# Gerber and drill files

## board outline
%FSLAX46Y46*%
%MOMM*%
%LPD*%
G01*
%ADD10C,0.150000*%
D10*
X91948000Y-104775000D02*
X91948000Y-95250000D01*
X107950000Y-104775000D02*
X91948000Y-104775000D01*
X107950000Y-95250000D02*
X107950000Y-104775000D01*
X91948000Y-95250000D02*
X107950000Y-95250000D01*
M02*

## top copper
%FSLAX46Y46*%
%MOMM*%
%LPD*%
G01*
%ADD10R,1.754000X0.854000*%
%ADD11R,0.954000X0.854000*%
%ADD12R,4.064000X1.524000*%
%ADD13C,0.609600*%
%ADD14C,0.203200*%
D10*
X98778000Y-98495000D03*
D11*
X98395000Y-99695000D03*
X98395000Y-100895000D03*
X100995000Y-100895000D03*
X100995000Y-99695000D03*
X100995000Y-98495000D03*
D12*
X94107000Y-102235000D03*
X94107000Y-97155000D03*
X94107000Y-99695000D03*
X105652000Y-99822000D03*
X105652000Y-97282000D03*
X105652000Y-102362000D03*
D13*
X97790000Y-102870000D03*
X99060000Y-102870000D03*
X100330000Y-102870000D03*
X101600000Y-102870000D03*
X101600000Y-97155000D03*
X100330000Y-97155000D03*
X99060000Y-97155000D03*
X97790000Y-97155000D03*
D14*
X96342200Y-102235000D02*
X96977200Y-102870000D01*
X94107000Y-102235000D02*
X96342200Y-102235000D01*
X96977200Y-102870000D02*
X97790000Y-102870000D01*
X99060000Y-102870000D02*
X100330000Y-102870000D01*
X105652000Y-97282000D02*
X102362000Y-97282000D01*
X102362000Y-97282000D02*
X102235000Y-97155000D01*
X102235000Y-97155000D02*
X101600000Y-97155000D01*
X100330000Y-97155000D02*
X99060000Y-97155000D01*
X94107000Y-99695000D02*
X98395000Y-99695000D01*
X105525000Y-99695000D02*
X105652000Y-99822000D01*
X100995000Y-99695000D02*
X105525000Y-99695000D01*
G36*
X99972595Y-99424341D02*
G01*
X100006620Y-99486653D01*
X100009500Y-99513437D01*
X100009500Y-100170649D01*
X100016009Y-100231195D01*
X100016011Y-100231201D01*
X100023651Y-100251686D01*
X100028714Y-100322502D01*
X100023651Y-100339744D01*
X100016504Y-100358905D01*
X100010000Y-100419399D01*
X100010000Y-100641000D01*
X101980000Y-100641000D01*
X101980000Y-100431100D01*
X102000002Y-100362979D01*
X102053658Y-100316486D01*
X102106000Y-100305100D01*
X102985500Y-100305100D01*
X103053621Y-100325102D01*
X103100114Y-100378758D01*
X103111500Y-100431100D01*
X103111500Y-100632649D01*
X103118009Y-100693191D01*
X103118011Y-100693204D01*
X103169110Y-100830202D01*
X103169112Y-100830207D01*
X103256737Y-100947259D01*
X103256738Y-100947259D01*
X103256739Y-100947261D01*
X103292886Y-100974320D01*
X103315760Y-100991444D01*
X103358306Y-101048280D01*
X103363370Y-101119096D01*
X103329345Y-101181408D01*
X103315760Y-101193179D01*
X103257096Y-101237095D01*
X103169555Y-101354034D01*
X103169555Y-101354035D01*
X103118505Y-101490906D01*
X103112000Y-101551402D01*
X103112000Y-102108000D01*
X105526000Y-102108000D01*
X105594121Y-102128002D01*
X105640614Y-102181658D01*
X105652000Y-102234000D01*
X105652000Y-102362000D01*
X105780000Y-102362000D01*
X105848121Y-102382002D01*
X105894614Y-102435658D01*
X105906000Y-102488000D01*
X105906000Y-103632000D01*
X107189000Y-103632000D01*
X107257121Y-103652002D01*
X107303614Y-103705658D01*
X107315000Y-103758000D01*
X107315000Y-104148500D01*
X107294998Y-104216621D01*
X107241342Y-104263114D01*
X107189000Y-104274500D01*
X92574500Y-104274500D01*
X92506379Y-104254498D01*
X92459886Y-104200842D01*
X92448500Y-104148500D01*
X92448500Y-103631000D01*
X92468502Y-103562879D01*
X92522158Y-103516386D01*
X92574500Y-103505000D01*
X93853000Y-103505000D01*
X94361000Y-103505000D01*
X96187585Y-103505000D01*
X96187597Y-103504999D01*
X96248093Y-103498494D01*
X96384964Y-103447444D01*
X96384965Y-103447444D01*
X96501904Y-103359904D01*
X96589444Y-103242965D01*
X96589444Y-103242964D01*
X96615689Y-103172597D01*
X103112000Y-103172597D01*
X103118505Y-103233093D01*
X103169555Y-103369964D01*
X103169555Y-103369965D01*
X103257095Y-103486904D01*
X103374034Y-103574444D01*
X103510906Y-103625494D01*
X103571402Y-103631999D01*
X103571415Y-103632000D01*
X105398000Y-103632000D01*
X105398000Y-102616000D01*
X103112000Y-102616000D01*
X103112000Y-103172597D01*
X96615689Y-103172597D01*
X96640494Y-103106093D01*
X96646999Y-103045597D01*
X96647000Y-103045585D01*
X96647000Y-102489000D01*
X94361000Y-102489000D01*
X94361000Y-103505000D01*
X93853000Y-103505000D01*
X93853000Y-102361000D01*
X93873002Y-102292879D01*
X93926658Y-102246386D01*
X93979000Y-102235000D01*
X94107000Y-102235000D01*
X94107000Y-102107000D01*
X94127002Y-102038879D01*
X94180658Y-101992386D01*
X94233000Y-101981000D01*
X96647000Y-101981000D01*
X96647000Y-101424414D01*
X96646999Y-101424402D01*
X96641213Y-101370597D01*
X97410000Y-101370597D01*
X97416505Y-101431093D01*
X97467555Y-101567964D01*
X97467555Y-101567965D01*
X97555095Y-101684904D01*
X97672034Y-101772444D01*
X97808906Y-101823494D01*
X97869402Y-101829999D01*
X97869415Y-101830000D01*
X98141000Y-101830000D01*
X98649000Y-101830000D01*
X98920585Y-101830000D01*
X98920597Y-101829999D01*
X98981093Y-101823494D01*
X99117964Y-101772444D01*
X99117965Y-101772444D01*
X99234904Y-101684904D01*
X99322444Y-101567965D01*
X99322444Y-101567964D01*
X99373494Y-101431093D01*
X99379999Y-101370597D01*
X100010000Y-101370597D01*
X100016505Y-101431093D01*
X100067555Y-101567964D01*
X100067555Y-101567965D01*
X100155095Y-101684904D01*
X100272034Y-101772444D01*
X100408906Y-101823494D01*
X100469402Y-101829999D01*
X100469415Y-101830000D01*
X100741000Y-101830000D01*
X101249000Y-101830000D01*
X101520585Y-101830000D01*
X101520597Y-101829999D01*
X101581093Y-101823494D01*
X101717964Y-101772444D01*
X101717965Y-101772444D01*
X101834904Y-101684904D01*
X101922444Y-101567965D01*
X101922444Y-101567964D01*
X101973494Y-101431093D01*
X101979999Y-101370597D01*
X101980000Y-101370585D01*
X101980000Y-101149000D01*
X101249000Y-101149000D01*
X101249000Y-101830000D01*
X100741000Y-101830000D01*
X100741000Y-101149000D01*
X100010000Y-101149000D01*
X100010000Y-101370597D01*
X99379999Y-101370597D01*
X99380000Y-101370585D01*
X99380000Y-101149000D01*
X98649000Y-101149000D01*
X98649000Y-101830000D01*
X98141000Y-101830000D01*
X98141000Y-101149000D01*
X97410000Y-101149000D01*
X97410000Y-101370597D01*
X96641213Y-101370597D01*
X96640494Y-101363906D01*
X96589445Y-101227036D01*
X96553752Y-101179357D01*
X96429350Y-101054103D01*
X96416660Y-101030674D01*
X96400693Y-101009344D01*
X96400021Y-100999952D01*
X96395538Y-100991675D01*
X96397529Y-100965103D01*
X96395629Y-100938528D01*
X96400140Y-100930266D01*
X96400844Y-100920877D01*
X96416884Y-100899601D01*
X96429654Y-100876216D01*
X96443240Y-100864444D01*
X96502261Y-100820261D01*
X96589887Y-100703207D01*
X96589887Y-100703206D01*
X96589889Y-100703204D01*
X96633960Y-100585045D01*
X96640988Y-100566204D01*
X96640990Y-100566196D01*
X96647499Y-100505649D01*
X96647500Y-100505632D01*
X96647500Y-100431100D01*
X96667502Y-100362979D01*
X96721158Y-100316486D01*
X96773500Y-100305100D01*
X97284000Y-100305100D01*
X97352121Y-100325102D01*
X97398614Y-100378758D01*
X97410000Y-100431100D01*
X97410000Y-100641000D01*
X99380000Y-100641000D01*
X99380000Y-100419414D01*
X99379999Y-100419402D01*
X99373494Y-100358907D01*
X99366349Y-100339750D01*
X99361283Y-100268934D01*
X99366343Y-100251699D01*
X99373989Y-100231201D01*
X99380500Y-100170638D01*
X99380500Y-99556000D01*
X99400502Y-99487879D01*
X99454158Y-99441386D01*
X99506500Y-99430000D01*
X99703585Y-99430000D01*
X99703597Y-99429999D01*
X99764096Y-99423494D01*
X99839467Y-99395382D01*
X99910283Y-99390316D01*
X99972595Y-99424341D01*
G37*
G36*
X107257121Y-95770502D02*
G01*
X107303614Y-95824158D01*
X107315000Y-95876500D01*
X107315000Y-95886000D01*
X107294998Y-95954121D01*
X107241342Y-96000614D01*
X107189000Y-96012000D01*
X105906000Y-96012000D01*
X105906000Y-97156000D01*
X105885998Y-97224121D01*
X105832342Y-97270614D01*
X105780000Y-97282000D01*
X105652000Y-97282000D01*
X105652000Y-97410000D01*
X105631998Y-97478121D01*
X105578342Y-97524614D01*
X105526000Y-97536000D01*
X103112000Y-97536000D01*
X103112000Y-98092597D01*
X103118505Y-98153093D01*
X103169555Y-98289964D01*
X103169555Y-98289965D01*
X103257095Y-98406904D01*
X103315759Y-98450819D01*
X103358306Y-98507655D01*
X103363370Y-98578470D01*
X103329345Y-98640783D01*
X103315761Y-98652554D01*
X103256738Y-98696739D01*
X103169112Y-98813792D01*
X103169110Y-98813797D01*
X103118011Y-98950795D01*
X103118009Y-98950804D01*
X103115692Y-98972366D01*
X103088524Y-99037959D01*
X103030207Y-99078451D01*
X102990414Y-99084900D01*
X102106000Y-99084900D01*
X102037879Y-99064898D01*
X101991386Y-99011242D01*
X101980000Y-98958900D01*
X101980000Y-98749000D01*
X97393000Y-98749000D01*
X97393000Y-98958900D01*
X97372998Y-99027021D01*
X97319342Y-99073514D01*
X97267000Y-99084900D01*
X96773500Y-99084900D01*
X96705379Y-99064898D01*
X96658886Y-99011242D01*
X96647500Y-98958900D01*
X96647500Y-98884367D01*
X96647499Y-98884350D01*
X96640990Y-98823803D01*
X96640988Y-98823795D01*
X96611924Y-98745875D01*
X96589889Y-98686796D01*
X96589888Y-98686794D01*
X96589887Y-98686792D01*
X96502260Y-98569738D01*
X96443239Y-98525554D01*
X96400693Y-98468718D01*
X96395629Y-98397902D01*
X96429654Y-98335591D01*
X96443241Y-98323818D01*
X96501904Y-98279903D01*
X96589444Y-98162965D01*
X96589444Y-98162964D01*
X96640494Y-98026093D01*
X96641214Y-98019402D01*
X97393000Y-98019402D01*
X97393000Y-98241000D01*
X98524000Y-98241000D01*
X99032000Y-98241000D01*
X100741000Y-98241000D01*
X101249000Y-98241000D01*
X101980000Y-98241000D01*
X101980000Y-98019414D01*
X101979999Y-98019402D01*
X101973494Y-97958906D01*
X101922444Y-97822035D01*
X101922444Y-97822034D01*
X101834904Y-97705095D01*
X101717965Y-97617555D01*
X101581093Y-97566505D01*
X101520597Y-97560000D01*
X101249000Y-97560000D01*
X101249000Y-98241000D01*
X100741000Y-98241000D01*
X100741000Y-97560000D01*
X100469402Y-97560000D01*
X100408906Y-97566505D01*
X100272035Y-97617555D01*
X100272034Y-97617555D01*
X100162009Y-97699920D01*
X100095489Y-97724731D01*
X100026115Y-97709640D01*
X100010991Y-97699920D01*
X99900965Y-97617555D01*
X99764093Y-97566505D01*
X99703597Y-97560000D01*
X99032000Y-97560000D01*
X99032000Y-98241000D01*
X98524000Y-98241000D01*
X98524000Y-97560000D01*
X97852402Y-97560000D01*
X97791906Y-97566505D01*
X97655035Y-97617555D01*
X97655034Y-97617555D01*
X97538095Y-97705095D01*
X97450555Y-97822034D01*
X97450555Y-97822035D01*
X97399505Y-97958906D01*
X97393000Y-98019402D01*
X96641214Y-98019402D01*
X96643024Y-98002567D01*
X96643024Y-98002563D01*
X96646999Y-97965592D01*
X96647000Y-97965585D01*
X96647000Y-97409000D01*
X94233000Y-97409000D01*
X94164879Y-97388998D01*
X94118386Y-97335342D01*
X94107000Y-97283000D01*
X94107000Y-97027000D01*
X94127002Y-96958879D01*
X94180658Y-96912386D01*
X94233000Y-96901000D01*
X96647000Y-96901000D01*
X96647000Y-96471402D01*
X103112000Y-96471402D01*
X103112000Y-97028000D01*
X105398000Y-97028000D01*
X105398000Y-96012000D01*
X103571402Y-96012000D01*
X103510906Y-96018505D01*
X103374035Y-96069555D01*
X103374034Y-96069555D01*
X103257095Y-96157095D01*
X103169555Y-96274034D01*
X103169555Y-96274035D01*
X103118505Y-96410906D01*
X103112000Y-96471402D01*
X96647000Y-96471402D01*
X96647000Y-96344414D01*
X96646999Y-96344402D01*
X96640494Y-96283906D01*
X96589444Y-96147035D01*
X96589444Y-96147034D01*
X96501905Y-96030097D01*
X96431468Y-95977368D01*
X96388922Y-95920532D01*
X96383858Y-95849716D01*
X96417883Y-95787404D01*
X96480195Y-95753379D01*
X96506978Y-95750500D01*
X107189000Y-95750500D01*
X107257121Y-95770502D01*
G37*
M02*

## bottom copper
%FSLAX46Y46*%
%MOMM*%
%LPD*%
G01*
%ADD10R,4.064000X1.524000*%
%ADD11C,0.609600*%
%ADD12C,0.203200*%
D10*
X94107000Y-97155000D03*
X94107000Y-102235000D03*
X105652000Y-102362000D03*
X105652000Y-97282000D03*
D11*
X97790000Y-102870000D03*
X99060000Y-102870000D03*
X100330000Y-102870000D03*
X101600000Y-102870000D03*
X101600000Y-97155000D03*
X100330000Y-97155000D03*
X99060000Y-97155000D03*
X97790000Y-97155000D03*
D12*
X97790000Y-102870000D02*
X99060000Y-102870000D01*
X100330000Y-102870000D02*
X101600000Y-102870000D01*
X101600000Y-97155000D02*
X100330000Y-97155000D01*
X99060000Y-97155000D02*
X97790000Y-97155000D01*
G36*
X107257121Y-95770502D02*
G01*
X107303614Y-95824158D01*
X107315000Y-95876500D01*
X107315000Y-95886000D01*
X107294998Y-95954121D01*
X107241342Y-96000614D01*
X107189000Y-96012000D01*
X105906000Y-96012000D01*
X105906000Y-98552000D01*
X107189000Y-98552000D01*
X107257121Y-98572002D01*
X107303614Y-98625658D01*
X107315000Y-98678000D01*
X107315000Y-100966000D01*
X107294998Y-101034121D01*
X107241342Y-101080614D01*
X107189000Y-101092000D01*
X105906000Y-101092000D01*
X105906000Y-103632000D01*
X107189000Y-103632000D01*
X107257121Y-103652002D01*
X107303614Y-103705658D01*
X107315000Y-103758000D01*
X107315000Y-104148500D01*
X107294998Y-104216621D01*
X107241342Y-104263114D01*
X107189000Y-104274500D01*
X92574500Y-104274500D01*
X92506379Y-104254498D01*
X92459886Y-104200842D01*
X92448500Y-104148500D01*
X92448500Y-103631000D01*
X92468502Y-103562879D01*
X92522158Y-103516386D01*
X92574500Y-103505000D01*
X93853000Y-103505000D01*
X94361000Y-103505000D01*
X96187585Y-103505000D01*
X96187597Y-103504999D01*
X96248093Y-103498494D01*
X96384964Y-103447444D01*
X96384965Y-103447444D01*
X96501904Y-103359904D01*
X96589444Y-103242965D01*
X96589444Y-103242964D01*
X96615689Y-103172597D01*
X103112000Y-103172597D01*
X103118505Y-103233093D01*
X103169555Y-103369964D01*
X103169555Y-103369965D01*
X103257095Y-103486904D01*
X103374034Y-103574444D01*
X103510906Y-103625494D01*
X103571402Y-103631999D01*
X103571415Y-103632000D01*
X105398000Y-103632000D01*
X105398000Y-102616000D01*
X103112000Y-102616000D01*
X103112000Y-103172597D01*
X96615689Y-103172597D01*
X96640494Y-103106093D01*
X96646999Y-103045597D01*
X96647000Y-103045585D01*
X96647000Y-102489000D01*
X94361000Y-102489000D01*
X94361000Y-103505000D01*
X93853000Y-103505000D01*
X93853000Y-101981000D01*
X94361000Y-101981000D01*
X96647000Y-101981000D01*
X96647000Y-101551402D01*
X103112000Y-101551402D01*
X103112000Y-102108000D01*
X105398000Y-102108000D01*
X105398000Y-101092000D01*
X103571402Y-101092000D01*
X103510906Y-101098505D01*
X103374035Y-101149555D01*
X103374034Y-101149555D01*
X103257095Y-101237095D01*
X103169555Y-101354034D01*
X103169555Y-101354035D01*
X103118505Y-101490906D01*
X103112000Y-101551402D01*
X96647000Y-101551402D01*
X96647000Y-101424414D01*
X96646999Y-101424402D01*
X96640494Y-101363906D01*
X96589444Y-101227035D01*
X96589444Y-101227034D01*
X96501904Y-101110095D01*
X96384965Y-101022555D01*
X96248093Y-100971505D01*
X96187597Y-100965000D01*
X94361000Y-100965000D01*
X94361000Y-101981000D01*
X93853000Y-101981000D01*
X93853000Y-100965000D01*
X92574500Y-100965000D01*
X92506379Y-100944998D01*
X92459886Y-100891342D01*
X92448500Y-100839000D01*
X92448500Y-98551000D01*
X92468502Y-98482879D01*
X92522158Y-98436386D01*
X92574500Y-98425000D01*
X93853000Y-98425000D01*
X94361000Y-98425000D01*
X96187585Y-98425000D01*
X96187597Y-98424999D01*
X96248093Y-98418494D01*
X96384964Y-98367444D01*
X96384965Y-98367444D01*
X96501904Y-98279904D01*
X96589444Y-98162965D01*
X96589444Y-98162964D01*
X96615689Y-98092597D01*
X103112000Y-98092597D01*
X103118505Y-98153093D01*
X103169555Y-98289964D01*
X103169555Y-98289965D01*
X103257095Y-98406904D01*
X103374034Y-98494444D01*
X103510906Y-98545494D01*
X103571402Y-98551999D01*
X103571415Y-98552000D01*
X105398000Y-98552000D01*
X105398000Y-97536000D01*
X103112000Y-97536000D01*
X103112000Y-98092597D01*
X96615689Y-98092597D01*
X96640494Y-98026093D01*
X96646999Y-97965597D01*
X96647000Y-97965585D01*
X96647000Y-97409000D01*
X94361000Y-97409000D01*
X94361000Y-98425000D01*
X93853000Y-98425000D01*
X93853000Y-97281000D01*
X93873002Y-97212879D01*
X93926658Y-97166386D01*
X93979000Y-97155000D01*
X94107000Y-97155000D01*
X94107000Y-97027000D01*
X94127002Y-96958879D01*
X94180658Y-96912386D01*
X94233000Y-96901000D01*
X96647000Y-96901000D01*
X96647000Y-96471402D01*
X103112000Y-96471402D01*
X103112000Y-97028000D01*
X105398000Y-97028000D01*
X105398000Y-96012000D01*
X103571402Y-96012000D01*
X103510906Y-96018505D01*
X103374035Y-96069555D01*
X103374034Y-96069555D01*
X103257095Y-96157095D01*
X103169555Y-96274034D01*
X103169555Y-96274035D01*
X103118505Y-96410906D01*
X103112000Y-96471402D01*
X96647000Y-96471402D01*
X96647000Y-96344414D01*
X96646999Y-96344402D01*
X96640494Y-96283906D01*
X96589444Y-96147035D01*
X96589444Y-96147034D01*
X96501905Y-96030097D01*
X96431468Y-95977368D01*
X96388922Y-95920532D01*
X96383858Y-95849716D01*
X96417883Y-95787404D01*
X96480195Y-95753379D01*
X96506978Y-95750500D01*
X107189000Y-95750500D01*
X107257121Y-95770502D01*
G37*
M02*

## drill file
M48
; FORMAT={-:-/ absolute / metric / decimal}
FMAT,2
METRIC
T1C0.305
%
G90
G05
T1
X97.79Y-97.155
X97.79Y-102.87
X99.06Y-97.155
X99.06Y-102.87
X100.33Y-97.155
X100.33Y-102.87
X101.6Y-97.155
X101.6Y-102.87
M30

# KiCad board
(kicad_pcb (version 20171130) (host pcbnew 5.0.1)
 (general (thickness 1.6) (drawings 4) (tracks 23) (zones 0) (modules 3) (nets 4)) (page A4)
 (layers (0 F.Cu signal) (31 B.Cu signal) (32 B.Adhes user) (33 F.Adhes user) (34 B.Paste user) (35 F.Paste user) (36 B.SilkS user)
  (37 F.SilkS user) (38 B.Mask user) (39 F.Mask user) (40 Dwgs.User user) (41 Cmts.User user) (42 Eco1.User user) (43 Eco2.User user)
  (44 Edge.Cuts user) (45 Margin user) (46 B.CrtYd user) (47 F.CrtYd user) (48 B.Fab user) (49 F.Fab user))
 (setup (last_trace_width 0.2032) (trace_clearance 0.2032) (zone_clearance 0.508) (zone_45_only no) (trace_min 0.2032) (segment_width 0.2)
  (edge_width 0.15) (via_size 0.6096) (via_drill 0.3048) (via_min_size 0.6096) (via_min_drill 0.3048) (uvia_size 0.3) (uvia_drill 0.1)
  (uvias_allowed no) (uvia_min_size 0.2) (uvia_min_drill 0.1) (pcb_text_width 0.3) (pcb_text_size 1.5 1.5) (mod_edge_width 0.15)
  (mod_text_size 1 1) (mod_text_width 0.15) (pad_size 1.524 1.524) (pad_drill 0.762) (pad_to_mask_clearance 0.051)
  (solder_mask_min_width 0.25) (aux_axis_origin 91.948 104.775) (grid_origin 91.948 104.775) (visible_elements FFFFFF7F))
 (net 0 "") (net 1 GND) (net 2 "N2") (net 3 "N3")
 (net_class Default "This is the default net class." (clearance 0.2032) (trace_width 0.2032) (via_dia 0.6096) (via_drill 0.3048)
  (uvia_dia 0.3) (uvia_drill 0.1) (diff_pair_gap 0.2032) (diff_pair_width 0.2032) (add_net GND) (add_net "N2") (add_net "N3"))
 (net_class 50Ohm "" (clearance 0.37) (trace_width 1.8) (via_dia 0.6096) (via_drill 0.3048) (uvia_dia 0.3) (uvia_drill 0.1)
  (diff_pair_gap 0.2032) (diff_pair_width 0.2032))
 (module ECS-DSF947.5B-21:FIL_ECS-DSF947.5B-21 (layer F.Cu) (at 99.695 99.695)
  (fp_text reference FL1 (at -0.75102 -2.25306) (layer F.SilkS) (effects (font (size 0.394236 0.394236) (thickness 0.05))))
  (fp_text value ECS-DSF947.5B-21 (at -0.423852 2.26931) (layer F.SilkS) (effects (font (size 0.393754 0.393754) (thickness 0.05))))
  (pad 1 smd rect (at -0.917 -1.2) (size 1.754 0.854) (layers F.Cu F.Paste F.Mask) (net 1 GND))
  (pad 2 smd rect (at -1.3 0) (size 0.954 0.854) (layers F.Cu F.Paste F.Mask) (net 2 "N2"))
  (pad 3 smd rect (at -1.3 1.2) (size 0.954 0.854) (layers F.Cu F.Paste F.Mask) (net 1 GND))
  (pad 4 smd rect (at 1.3 1.2) (size 0.954 0.854) (layers F.Cu F.Paste F.Mask) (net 1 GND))
  (pad 5 smd rect (at 1.3 0) (size 0.954 0.854) (layers F.Cu F.Paste F.Mask) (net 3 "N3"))
  (pad 6 smd rect (at 1.3 -1.2) (size 0.954 0.854) (layers F.Cu F.Paste F.Mask) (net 1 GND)))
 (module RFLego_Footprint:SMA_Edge (layer F.Cu) (at 92.075 99.695)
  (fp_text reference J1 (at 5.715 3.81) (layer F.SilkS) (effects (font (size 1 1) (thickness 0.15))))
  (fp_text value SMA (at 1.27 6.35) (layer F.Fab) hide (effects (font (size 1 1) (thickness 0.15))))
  (pad 2 smd rect (at 2.032 2.54) (size 4.064 1.524) (layers F.Cu F.Mask) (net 1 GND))
  (pad 2 smd rect (at 2.032 -2.54) (size 4.064 1.524) (layers B.Cu B.Mask) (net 1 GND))
  (pad 2 smd rect (at 2.032 2.54) (size 4.064 1.524) (layers B.Cu B.Mask) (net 1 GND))
  (pad 2 smd rect (at 2.032 -2.54) (size 4.064 1.524) (layers F.Cu F.Mask) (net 1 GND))
  (pad 1 smd rect (at 2.032 0) (size 4.064 1.524) (layers F.Cu F.Mask) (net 2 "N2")))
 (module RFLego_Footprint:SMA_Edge (layer F.Cu) (at 103.62 99.822)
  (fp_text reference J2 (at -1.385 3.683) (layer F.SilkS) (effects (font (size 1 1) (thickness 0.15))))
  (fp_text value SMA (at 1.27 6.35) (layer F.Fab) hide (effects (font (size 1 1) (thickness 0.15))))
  (pad 1 smd rect (at 2.032 0) (size 4.064 1.524) (layers F.Cu F.Mask) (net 3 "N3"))
  (pad 2 smd rect (at 2.032 -2.54) (size 4.064 1.524) (layers F.Cu F.Mask) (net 1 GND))
  (pad 2 smd rect (at 2.032 2.54) (size 4.064 1.524) (layers B.Cu B.Mask) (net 1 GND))
  (pad 2 smd rect (at 2.032 -2.54) (size 4.064 1.524) (layers B.Cu B.Mask) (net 1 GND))
  (pad 2 smd rect (at 2.032 2.54) (size 4.064 1.524) (layers F.Cu F.Mask) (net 1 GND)))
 (gr_line (start 91.948 104.775) (end 91.948 95.25) (layer Edge.Cuts) (width 0.15))
 (gr_line (start 107.95 104.775) (end 91.948 104.775) (layer Edge.Cuts) (width 0.15))
 (gr_line (start 107.95 95.25) (end 107.95 104.775) (layer Edge.Cuts) (width 0.15))
 (gr_line (start 91.948 95.25) (end 107.95 95.25) (layer Edge.Cuts) (width 0.15))
 (segment (start 96.3422 102.235) (end 96.9772 102.87) (width 0.2032) (layer F.Cu) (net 1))
 (segment (start 94.107 102.235) (end 96.3422 102.235) (width 0.2032) (layer F.Cu) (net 1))
 (via (at 97.79 102.87) (size 0.6096) (drill 0.3048) (layers F.Cu B.Cu) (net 1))
 (segment (start 96.9772 102.87) (end 97.79 102.87) (width 0.2032) (layer F.Cu) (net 1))
 (via (at 99.06 102.87) (size 0.6096) (drill 0.3048) (layers F.Cu B.Cu) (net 1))
 (segment (start 97.79 102.87) (end 99.06 102.87) (width 0.2032) (layer B.Cu) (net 1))
 (via (at 100.33 102.87) (size 0.6096) (drill 0.3048) (layers F.Cu B.Cu) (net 1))
 (segment (start 99.06 102.87) (end 100.33 102.87) (width 0.2032) (layer F.Cu) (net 1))
 (via (at 101.6 102.87) (size 0.6096) (drill 0.3048) (layers F.Cu B.Cu) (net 1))
 (segment (start 100.33 102.87) (end 101.6 102.87) (width 0.2032) (layer B.Cu) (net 1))
 (segment (start 105.652 97.282) (end 102.362 97.282) (width 0.2032) (layer F.Cu) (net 1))
 (segment (start 102.362 97.282) (end 102.235 97.155) (width 0.2032) (layer F.Cu) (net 1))
 (via (at 101.6 97.155) (size 0.6096) (drill 0.3048) (layers F.Cu B.Cu) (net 1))
 (segment (start 102.235 97.155) (end 101.6 97.155) (width 0.2032) (layer F.Cu) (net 1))
 (via (at 100.33 97.155) (size 0.6096) (drill 0.3048) (layers F.Cu B.Cu) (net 1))
 (segment (start 101.6 97.155) (end 100.33 97.155) (width 0.2032) (layer B.Cu) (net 1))
 (via (at 99.06 97.155) (size 0.6096) (drill 0.3048) (layers F.Cu B.Cu) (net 1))
 (segment (start 100.33 97.155) (end 99.06 97.155) (width 0.2032) (layer F.Cu) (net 1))
 (via (at 97.79 97.155) (size 0.6096) (drill 0.3048) (layers F.Cu B.Cu) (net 1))
 (segment (start 99.06 97.155) (end 97.79 97.155) (width 0.2032) (layer B.Cu) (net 1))
 (segment (start 94.107 99.695) (end 98.395 99.695) (width 0.2032) (layer F.Cu) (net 2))
 (segment (start 105.525 99.695) (end 105.652 99.822) (width 0.2032) (layer F.Cu) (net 3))
 (segment (start 100.995 99.695) (end 105.525 99.695) (width 0.2032) (layer F.Cu) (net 3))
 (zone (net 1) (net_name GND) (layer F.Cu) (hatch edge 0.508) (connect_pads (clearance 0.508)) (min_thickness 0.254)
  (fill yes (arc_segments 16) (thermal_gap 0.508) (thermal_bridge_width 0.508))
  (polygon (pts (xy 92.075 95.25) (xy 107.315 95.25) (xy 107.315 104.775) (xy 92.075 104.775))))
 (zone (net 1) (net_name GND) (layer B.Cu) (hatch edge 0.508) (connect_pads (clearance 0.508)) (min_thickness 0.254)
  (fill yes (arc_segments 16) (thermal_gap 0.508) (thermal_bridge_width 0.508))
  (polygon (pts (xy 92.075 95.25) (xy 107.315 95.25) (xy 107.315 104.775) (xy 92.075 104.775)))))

